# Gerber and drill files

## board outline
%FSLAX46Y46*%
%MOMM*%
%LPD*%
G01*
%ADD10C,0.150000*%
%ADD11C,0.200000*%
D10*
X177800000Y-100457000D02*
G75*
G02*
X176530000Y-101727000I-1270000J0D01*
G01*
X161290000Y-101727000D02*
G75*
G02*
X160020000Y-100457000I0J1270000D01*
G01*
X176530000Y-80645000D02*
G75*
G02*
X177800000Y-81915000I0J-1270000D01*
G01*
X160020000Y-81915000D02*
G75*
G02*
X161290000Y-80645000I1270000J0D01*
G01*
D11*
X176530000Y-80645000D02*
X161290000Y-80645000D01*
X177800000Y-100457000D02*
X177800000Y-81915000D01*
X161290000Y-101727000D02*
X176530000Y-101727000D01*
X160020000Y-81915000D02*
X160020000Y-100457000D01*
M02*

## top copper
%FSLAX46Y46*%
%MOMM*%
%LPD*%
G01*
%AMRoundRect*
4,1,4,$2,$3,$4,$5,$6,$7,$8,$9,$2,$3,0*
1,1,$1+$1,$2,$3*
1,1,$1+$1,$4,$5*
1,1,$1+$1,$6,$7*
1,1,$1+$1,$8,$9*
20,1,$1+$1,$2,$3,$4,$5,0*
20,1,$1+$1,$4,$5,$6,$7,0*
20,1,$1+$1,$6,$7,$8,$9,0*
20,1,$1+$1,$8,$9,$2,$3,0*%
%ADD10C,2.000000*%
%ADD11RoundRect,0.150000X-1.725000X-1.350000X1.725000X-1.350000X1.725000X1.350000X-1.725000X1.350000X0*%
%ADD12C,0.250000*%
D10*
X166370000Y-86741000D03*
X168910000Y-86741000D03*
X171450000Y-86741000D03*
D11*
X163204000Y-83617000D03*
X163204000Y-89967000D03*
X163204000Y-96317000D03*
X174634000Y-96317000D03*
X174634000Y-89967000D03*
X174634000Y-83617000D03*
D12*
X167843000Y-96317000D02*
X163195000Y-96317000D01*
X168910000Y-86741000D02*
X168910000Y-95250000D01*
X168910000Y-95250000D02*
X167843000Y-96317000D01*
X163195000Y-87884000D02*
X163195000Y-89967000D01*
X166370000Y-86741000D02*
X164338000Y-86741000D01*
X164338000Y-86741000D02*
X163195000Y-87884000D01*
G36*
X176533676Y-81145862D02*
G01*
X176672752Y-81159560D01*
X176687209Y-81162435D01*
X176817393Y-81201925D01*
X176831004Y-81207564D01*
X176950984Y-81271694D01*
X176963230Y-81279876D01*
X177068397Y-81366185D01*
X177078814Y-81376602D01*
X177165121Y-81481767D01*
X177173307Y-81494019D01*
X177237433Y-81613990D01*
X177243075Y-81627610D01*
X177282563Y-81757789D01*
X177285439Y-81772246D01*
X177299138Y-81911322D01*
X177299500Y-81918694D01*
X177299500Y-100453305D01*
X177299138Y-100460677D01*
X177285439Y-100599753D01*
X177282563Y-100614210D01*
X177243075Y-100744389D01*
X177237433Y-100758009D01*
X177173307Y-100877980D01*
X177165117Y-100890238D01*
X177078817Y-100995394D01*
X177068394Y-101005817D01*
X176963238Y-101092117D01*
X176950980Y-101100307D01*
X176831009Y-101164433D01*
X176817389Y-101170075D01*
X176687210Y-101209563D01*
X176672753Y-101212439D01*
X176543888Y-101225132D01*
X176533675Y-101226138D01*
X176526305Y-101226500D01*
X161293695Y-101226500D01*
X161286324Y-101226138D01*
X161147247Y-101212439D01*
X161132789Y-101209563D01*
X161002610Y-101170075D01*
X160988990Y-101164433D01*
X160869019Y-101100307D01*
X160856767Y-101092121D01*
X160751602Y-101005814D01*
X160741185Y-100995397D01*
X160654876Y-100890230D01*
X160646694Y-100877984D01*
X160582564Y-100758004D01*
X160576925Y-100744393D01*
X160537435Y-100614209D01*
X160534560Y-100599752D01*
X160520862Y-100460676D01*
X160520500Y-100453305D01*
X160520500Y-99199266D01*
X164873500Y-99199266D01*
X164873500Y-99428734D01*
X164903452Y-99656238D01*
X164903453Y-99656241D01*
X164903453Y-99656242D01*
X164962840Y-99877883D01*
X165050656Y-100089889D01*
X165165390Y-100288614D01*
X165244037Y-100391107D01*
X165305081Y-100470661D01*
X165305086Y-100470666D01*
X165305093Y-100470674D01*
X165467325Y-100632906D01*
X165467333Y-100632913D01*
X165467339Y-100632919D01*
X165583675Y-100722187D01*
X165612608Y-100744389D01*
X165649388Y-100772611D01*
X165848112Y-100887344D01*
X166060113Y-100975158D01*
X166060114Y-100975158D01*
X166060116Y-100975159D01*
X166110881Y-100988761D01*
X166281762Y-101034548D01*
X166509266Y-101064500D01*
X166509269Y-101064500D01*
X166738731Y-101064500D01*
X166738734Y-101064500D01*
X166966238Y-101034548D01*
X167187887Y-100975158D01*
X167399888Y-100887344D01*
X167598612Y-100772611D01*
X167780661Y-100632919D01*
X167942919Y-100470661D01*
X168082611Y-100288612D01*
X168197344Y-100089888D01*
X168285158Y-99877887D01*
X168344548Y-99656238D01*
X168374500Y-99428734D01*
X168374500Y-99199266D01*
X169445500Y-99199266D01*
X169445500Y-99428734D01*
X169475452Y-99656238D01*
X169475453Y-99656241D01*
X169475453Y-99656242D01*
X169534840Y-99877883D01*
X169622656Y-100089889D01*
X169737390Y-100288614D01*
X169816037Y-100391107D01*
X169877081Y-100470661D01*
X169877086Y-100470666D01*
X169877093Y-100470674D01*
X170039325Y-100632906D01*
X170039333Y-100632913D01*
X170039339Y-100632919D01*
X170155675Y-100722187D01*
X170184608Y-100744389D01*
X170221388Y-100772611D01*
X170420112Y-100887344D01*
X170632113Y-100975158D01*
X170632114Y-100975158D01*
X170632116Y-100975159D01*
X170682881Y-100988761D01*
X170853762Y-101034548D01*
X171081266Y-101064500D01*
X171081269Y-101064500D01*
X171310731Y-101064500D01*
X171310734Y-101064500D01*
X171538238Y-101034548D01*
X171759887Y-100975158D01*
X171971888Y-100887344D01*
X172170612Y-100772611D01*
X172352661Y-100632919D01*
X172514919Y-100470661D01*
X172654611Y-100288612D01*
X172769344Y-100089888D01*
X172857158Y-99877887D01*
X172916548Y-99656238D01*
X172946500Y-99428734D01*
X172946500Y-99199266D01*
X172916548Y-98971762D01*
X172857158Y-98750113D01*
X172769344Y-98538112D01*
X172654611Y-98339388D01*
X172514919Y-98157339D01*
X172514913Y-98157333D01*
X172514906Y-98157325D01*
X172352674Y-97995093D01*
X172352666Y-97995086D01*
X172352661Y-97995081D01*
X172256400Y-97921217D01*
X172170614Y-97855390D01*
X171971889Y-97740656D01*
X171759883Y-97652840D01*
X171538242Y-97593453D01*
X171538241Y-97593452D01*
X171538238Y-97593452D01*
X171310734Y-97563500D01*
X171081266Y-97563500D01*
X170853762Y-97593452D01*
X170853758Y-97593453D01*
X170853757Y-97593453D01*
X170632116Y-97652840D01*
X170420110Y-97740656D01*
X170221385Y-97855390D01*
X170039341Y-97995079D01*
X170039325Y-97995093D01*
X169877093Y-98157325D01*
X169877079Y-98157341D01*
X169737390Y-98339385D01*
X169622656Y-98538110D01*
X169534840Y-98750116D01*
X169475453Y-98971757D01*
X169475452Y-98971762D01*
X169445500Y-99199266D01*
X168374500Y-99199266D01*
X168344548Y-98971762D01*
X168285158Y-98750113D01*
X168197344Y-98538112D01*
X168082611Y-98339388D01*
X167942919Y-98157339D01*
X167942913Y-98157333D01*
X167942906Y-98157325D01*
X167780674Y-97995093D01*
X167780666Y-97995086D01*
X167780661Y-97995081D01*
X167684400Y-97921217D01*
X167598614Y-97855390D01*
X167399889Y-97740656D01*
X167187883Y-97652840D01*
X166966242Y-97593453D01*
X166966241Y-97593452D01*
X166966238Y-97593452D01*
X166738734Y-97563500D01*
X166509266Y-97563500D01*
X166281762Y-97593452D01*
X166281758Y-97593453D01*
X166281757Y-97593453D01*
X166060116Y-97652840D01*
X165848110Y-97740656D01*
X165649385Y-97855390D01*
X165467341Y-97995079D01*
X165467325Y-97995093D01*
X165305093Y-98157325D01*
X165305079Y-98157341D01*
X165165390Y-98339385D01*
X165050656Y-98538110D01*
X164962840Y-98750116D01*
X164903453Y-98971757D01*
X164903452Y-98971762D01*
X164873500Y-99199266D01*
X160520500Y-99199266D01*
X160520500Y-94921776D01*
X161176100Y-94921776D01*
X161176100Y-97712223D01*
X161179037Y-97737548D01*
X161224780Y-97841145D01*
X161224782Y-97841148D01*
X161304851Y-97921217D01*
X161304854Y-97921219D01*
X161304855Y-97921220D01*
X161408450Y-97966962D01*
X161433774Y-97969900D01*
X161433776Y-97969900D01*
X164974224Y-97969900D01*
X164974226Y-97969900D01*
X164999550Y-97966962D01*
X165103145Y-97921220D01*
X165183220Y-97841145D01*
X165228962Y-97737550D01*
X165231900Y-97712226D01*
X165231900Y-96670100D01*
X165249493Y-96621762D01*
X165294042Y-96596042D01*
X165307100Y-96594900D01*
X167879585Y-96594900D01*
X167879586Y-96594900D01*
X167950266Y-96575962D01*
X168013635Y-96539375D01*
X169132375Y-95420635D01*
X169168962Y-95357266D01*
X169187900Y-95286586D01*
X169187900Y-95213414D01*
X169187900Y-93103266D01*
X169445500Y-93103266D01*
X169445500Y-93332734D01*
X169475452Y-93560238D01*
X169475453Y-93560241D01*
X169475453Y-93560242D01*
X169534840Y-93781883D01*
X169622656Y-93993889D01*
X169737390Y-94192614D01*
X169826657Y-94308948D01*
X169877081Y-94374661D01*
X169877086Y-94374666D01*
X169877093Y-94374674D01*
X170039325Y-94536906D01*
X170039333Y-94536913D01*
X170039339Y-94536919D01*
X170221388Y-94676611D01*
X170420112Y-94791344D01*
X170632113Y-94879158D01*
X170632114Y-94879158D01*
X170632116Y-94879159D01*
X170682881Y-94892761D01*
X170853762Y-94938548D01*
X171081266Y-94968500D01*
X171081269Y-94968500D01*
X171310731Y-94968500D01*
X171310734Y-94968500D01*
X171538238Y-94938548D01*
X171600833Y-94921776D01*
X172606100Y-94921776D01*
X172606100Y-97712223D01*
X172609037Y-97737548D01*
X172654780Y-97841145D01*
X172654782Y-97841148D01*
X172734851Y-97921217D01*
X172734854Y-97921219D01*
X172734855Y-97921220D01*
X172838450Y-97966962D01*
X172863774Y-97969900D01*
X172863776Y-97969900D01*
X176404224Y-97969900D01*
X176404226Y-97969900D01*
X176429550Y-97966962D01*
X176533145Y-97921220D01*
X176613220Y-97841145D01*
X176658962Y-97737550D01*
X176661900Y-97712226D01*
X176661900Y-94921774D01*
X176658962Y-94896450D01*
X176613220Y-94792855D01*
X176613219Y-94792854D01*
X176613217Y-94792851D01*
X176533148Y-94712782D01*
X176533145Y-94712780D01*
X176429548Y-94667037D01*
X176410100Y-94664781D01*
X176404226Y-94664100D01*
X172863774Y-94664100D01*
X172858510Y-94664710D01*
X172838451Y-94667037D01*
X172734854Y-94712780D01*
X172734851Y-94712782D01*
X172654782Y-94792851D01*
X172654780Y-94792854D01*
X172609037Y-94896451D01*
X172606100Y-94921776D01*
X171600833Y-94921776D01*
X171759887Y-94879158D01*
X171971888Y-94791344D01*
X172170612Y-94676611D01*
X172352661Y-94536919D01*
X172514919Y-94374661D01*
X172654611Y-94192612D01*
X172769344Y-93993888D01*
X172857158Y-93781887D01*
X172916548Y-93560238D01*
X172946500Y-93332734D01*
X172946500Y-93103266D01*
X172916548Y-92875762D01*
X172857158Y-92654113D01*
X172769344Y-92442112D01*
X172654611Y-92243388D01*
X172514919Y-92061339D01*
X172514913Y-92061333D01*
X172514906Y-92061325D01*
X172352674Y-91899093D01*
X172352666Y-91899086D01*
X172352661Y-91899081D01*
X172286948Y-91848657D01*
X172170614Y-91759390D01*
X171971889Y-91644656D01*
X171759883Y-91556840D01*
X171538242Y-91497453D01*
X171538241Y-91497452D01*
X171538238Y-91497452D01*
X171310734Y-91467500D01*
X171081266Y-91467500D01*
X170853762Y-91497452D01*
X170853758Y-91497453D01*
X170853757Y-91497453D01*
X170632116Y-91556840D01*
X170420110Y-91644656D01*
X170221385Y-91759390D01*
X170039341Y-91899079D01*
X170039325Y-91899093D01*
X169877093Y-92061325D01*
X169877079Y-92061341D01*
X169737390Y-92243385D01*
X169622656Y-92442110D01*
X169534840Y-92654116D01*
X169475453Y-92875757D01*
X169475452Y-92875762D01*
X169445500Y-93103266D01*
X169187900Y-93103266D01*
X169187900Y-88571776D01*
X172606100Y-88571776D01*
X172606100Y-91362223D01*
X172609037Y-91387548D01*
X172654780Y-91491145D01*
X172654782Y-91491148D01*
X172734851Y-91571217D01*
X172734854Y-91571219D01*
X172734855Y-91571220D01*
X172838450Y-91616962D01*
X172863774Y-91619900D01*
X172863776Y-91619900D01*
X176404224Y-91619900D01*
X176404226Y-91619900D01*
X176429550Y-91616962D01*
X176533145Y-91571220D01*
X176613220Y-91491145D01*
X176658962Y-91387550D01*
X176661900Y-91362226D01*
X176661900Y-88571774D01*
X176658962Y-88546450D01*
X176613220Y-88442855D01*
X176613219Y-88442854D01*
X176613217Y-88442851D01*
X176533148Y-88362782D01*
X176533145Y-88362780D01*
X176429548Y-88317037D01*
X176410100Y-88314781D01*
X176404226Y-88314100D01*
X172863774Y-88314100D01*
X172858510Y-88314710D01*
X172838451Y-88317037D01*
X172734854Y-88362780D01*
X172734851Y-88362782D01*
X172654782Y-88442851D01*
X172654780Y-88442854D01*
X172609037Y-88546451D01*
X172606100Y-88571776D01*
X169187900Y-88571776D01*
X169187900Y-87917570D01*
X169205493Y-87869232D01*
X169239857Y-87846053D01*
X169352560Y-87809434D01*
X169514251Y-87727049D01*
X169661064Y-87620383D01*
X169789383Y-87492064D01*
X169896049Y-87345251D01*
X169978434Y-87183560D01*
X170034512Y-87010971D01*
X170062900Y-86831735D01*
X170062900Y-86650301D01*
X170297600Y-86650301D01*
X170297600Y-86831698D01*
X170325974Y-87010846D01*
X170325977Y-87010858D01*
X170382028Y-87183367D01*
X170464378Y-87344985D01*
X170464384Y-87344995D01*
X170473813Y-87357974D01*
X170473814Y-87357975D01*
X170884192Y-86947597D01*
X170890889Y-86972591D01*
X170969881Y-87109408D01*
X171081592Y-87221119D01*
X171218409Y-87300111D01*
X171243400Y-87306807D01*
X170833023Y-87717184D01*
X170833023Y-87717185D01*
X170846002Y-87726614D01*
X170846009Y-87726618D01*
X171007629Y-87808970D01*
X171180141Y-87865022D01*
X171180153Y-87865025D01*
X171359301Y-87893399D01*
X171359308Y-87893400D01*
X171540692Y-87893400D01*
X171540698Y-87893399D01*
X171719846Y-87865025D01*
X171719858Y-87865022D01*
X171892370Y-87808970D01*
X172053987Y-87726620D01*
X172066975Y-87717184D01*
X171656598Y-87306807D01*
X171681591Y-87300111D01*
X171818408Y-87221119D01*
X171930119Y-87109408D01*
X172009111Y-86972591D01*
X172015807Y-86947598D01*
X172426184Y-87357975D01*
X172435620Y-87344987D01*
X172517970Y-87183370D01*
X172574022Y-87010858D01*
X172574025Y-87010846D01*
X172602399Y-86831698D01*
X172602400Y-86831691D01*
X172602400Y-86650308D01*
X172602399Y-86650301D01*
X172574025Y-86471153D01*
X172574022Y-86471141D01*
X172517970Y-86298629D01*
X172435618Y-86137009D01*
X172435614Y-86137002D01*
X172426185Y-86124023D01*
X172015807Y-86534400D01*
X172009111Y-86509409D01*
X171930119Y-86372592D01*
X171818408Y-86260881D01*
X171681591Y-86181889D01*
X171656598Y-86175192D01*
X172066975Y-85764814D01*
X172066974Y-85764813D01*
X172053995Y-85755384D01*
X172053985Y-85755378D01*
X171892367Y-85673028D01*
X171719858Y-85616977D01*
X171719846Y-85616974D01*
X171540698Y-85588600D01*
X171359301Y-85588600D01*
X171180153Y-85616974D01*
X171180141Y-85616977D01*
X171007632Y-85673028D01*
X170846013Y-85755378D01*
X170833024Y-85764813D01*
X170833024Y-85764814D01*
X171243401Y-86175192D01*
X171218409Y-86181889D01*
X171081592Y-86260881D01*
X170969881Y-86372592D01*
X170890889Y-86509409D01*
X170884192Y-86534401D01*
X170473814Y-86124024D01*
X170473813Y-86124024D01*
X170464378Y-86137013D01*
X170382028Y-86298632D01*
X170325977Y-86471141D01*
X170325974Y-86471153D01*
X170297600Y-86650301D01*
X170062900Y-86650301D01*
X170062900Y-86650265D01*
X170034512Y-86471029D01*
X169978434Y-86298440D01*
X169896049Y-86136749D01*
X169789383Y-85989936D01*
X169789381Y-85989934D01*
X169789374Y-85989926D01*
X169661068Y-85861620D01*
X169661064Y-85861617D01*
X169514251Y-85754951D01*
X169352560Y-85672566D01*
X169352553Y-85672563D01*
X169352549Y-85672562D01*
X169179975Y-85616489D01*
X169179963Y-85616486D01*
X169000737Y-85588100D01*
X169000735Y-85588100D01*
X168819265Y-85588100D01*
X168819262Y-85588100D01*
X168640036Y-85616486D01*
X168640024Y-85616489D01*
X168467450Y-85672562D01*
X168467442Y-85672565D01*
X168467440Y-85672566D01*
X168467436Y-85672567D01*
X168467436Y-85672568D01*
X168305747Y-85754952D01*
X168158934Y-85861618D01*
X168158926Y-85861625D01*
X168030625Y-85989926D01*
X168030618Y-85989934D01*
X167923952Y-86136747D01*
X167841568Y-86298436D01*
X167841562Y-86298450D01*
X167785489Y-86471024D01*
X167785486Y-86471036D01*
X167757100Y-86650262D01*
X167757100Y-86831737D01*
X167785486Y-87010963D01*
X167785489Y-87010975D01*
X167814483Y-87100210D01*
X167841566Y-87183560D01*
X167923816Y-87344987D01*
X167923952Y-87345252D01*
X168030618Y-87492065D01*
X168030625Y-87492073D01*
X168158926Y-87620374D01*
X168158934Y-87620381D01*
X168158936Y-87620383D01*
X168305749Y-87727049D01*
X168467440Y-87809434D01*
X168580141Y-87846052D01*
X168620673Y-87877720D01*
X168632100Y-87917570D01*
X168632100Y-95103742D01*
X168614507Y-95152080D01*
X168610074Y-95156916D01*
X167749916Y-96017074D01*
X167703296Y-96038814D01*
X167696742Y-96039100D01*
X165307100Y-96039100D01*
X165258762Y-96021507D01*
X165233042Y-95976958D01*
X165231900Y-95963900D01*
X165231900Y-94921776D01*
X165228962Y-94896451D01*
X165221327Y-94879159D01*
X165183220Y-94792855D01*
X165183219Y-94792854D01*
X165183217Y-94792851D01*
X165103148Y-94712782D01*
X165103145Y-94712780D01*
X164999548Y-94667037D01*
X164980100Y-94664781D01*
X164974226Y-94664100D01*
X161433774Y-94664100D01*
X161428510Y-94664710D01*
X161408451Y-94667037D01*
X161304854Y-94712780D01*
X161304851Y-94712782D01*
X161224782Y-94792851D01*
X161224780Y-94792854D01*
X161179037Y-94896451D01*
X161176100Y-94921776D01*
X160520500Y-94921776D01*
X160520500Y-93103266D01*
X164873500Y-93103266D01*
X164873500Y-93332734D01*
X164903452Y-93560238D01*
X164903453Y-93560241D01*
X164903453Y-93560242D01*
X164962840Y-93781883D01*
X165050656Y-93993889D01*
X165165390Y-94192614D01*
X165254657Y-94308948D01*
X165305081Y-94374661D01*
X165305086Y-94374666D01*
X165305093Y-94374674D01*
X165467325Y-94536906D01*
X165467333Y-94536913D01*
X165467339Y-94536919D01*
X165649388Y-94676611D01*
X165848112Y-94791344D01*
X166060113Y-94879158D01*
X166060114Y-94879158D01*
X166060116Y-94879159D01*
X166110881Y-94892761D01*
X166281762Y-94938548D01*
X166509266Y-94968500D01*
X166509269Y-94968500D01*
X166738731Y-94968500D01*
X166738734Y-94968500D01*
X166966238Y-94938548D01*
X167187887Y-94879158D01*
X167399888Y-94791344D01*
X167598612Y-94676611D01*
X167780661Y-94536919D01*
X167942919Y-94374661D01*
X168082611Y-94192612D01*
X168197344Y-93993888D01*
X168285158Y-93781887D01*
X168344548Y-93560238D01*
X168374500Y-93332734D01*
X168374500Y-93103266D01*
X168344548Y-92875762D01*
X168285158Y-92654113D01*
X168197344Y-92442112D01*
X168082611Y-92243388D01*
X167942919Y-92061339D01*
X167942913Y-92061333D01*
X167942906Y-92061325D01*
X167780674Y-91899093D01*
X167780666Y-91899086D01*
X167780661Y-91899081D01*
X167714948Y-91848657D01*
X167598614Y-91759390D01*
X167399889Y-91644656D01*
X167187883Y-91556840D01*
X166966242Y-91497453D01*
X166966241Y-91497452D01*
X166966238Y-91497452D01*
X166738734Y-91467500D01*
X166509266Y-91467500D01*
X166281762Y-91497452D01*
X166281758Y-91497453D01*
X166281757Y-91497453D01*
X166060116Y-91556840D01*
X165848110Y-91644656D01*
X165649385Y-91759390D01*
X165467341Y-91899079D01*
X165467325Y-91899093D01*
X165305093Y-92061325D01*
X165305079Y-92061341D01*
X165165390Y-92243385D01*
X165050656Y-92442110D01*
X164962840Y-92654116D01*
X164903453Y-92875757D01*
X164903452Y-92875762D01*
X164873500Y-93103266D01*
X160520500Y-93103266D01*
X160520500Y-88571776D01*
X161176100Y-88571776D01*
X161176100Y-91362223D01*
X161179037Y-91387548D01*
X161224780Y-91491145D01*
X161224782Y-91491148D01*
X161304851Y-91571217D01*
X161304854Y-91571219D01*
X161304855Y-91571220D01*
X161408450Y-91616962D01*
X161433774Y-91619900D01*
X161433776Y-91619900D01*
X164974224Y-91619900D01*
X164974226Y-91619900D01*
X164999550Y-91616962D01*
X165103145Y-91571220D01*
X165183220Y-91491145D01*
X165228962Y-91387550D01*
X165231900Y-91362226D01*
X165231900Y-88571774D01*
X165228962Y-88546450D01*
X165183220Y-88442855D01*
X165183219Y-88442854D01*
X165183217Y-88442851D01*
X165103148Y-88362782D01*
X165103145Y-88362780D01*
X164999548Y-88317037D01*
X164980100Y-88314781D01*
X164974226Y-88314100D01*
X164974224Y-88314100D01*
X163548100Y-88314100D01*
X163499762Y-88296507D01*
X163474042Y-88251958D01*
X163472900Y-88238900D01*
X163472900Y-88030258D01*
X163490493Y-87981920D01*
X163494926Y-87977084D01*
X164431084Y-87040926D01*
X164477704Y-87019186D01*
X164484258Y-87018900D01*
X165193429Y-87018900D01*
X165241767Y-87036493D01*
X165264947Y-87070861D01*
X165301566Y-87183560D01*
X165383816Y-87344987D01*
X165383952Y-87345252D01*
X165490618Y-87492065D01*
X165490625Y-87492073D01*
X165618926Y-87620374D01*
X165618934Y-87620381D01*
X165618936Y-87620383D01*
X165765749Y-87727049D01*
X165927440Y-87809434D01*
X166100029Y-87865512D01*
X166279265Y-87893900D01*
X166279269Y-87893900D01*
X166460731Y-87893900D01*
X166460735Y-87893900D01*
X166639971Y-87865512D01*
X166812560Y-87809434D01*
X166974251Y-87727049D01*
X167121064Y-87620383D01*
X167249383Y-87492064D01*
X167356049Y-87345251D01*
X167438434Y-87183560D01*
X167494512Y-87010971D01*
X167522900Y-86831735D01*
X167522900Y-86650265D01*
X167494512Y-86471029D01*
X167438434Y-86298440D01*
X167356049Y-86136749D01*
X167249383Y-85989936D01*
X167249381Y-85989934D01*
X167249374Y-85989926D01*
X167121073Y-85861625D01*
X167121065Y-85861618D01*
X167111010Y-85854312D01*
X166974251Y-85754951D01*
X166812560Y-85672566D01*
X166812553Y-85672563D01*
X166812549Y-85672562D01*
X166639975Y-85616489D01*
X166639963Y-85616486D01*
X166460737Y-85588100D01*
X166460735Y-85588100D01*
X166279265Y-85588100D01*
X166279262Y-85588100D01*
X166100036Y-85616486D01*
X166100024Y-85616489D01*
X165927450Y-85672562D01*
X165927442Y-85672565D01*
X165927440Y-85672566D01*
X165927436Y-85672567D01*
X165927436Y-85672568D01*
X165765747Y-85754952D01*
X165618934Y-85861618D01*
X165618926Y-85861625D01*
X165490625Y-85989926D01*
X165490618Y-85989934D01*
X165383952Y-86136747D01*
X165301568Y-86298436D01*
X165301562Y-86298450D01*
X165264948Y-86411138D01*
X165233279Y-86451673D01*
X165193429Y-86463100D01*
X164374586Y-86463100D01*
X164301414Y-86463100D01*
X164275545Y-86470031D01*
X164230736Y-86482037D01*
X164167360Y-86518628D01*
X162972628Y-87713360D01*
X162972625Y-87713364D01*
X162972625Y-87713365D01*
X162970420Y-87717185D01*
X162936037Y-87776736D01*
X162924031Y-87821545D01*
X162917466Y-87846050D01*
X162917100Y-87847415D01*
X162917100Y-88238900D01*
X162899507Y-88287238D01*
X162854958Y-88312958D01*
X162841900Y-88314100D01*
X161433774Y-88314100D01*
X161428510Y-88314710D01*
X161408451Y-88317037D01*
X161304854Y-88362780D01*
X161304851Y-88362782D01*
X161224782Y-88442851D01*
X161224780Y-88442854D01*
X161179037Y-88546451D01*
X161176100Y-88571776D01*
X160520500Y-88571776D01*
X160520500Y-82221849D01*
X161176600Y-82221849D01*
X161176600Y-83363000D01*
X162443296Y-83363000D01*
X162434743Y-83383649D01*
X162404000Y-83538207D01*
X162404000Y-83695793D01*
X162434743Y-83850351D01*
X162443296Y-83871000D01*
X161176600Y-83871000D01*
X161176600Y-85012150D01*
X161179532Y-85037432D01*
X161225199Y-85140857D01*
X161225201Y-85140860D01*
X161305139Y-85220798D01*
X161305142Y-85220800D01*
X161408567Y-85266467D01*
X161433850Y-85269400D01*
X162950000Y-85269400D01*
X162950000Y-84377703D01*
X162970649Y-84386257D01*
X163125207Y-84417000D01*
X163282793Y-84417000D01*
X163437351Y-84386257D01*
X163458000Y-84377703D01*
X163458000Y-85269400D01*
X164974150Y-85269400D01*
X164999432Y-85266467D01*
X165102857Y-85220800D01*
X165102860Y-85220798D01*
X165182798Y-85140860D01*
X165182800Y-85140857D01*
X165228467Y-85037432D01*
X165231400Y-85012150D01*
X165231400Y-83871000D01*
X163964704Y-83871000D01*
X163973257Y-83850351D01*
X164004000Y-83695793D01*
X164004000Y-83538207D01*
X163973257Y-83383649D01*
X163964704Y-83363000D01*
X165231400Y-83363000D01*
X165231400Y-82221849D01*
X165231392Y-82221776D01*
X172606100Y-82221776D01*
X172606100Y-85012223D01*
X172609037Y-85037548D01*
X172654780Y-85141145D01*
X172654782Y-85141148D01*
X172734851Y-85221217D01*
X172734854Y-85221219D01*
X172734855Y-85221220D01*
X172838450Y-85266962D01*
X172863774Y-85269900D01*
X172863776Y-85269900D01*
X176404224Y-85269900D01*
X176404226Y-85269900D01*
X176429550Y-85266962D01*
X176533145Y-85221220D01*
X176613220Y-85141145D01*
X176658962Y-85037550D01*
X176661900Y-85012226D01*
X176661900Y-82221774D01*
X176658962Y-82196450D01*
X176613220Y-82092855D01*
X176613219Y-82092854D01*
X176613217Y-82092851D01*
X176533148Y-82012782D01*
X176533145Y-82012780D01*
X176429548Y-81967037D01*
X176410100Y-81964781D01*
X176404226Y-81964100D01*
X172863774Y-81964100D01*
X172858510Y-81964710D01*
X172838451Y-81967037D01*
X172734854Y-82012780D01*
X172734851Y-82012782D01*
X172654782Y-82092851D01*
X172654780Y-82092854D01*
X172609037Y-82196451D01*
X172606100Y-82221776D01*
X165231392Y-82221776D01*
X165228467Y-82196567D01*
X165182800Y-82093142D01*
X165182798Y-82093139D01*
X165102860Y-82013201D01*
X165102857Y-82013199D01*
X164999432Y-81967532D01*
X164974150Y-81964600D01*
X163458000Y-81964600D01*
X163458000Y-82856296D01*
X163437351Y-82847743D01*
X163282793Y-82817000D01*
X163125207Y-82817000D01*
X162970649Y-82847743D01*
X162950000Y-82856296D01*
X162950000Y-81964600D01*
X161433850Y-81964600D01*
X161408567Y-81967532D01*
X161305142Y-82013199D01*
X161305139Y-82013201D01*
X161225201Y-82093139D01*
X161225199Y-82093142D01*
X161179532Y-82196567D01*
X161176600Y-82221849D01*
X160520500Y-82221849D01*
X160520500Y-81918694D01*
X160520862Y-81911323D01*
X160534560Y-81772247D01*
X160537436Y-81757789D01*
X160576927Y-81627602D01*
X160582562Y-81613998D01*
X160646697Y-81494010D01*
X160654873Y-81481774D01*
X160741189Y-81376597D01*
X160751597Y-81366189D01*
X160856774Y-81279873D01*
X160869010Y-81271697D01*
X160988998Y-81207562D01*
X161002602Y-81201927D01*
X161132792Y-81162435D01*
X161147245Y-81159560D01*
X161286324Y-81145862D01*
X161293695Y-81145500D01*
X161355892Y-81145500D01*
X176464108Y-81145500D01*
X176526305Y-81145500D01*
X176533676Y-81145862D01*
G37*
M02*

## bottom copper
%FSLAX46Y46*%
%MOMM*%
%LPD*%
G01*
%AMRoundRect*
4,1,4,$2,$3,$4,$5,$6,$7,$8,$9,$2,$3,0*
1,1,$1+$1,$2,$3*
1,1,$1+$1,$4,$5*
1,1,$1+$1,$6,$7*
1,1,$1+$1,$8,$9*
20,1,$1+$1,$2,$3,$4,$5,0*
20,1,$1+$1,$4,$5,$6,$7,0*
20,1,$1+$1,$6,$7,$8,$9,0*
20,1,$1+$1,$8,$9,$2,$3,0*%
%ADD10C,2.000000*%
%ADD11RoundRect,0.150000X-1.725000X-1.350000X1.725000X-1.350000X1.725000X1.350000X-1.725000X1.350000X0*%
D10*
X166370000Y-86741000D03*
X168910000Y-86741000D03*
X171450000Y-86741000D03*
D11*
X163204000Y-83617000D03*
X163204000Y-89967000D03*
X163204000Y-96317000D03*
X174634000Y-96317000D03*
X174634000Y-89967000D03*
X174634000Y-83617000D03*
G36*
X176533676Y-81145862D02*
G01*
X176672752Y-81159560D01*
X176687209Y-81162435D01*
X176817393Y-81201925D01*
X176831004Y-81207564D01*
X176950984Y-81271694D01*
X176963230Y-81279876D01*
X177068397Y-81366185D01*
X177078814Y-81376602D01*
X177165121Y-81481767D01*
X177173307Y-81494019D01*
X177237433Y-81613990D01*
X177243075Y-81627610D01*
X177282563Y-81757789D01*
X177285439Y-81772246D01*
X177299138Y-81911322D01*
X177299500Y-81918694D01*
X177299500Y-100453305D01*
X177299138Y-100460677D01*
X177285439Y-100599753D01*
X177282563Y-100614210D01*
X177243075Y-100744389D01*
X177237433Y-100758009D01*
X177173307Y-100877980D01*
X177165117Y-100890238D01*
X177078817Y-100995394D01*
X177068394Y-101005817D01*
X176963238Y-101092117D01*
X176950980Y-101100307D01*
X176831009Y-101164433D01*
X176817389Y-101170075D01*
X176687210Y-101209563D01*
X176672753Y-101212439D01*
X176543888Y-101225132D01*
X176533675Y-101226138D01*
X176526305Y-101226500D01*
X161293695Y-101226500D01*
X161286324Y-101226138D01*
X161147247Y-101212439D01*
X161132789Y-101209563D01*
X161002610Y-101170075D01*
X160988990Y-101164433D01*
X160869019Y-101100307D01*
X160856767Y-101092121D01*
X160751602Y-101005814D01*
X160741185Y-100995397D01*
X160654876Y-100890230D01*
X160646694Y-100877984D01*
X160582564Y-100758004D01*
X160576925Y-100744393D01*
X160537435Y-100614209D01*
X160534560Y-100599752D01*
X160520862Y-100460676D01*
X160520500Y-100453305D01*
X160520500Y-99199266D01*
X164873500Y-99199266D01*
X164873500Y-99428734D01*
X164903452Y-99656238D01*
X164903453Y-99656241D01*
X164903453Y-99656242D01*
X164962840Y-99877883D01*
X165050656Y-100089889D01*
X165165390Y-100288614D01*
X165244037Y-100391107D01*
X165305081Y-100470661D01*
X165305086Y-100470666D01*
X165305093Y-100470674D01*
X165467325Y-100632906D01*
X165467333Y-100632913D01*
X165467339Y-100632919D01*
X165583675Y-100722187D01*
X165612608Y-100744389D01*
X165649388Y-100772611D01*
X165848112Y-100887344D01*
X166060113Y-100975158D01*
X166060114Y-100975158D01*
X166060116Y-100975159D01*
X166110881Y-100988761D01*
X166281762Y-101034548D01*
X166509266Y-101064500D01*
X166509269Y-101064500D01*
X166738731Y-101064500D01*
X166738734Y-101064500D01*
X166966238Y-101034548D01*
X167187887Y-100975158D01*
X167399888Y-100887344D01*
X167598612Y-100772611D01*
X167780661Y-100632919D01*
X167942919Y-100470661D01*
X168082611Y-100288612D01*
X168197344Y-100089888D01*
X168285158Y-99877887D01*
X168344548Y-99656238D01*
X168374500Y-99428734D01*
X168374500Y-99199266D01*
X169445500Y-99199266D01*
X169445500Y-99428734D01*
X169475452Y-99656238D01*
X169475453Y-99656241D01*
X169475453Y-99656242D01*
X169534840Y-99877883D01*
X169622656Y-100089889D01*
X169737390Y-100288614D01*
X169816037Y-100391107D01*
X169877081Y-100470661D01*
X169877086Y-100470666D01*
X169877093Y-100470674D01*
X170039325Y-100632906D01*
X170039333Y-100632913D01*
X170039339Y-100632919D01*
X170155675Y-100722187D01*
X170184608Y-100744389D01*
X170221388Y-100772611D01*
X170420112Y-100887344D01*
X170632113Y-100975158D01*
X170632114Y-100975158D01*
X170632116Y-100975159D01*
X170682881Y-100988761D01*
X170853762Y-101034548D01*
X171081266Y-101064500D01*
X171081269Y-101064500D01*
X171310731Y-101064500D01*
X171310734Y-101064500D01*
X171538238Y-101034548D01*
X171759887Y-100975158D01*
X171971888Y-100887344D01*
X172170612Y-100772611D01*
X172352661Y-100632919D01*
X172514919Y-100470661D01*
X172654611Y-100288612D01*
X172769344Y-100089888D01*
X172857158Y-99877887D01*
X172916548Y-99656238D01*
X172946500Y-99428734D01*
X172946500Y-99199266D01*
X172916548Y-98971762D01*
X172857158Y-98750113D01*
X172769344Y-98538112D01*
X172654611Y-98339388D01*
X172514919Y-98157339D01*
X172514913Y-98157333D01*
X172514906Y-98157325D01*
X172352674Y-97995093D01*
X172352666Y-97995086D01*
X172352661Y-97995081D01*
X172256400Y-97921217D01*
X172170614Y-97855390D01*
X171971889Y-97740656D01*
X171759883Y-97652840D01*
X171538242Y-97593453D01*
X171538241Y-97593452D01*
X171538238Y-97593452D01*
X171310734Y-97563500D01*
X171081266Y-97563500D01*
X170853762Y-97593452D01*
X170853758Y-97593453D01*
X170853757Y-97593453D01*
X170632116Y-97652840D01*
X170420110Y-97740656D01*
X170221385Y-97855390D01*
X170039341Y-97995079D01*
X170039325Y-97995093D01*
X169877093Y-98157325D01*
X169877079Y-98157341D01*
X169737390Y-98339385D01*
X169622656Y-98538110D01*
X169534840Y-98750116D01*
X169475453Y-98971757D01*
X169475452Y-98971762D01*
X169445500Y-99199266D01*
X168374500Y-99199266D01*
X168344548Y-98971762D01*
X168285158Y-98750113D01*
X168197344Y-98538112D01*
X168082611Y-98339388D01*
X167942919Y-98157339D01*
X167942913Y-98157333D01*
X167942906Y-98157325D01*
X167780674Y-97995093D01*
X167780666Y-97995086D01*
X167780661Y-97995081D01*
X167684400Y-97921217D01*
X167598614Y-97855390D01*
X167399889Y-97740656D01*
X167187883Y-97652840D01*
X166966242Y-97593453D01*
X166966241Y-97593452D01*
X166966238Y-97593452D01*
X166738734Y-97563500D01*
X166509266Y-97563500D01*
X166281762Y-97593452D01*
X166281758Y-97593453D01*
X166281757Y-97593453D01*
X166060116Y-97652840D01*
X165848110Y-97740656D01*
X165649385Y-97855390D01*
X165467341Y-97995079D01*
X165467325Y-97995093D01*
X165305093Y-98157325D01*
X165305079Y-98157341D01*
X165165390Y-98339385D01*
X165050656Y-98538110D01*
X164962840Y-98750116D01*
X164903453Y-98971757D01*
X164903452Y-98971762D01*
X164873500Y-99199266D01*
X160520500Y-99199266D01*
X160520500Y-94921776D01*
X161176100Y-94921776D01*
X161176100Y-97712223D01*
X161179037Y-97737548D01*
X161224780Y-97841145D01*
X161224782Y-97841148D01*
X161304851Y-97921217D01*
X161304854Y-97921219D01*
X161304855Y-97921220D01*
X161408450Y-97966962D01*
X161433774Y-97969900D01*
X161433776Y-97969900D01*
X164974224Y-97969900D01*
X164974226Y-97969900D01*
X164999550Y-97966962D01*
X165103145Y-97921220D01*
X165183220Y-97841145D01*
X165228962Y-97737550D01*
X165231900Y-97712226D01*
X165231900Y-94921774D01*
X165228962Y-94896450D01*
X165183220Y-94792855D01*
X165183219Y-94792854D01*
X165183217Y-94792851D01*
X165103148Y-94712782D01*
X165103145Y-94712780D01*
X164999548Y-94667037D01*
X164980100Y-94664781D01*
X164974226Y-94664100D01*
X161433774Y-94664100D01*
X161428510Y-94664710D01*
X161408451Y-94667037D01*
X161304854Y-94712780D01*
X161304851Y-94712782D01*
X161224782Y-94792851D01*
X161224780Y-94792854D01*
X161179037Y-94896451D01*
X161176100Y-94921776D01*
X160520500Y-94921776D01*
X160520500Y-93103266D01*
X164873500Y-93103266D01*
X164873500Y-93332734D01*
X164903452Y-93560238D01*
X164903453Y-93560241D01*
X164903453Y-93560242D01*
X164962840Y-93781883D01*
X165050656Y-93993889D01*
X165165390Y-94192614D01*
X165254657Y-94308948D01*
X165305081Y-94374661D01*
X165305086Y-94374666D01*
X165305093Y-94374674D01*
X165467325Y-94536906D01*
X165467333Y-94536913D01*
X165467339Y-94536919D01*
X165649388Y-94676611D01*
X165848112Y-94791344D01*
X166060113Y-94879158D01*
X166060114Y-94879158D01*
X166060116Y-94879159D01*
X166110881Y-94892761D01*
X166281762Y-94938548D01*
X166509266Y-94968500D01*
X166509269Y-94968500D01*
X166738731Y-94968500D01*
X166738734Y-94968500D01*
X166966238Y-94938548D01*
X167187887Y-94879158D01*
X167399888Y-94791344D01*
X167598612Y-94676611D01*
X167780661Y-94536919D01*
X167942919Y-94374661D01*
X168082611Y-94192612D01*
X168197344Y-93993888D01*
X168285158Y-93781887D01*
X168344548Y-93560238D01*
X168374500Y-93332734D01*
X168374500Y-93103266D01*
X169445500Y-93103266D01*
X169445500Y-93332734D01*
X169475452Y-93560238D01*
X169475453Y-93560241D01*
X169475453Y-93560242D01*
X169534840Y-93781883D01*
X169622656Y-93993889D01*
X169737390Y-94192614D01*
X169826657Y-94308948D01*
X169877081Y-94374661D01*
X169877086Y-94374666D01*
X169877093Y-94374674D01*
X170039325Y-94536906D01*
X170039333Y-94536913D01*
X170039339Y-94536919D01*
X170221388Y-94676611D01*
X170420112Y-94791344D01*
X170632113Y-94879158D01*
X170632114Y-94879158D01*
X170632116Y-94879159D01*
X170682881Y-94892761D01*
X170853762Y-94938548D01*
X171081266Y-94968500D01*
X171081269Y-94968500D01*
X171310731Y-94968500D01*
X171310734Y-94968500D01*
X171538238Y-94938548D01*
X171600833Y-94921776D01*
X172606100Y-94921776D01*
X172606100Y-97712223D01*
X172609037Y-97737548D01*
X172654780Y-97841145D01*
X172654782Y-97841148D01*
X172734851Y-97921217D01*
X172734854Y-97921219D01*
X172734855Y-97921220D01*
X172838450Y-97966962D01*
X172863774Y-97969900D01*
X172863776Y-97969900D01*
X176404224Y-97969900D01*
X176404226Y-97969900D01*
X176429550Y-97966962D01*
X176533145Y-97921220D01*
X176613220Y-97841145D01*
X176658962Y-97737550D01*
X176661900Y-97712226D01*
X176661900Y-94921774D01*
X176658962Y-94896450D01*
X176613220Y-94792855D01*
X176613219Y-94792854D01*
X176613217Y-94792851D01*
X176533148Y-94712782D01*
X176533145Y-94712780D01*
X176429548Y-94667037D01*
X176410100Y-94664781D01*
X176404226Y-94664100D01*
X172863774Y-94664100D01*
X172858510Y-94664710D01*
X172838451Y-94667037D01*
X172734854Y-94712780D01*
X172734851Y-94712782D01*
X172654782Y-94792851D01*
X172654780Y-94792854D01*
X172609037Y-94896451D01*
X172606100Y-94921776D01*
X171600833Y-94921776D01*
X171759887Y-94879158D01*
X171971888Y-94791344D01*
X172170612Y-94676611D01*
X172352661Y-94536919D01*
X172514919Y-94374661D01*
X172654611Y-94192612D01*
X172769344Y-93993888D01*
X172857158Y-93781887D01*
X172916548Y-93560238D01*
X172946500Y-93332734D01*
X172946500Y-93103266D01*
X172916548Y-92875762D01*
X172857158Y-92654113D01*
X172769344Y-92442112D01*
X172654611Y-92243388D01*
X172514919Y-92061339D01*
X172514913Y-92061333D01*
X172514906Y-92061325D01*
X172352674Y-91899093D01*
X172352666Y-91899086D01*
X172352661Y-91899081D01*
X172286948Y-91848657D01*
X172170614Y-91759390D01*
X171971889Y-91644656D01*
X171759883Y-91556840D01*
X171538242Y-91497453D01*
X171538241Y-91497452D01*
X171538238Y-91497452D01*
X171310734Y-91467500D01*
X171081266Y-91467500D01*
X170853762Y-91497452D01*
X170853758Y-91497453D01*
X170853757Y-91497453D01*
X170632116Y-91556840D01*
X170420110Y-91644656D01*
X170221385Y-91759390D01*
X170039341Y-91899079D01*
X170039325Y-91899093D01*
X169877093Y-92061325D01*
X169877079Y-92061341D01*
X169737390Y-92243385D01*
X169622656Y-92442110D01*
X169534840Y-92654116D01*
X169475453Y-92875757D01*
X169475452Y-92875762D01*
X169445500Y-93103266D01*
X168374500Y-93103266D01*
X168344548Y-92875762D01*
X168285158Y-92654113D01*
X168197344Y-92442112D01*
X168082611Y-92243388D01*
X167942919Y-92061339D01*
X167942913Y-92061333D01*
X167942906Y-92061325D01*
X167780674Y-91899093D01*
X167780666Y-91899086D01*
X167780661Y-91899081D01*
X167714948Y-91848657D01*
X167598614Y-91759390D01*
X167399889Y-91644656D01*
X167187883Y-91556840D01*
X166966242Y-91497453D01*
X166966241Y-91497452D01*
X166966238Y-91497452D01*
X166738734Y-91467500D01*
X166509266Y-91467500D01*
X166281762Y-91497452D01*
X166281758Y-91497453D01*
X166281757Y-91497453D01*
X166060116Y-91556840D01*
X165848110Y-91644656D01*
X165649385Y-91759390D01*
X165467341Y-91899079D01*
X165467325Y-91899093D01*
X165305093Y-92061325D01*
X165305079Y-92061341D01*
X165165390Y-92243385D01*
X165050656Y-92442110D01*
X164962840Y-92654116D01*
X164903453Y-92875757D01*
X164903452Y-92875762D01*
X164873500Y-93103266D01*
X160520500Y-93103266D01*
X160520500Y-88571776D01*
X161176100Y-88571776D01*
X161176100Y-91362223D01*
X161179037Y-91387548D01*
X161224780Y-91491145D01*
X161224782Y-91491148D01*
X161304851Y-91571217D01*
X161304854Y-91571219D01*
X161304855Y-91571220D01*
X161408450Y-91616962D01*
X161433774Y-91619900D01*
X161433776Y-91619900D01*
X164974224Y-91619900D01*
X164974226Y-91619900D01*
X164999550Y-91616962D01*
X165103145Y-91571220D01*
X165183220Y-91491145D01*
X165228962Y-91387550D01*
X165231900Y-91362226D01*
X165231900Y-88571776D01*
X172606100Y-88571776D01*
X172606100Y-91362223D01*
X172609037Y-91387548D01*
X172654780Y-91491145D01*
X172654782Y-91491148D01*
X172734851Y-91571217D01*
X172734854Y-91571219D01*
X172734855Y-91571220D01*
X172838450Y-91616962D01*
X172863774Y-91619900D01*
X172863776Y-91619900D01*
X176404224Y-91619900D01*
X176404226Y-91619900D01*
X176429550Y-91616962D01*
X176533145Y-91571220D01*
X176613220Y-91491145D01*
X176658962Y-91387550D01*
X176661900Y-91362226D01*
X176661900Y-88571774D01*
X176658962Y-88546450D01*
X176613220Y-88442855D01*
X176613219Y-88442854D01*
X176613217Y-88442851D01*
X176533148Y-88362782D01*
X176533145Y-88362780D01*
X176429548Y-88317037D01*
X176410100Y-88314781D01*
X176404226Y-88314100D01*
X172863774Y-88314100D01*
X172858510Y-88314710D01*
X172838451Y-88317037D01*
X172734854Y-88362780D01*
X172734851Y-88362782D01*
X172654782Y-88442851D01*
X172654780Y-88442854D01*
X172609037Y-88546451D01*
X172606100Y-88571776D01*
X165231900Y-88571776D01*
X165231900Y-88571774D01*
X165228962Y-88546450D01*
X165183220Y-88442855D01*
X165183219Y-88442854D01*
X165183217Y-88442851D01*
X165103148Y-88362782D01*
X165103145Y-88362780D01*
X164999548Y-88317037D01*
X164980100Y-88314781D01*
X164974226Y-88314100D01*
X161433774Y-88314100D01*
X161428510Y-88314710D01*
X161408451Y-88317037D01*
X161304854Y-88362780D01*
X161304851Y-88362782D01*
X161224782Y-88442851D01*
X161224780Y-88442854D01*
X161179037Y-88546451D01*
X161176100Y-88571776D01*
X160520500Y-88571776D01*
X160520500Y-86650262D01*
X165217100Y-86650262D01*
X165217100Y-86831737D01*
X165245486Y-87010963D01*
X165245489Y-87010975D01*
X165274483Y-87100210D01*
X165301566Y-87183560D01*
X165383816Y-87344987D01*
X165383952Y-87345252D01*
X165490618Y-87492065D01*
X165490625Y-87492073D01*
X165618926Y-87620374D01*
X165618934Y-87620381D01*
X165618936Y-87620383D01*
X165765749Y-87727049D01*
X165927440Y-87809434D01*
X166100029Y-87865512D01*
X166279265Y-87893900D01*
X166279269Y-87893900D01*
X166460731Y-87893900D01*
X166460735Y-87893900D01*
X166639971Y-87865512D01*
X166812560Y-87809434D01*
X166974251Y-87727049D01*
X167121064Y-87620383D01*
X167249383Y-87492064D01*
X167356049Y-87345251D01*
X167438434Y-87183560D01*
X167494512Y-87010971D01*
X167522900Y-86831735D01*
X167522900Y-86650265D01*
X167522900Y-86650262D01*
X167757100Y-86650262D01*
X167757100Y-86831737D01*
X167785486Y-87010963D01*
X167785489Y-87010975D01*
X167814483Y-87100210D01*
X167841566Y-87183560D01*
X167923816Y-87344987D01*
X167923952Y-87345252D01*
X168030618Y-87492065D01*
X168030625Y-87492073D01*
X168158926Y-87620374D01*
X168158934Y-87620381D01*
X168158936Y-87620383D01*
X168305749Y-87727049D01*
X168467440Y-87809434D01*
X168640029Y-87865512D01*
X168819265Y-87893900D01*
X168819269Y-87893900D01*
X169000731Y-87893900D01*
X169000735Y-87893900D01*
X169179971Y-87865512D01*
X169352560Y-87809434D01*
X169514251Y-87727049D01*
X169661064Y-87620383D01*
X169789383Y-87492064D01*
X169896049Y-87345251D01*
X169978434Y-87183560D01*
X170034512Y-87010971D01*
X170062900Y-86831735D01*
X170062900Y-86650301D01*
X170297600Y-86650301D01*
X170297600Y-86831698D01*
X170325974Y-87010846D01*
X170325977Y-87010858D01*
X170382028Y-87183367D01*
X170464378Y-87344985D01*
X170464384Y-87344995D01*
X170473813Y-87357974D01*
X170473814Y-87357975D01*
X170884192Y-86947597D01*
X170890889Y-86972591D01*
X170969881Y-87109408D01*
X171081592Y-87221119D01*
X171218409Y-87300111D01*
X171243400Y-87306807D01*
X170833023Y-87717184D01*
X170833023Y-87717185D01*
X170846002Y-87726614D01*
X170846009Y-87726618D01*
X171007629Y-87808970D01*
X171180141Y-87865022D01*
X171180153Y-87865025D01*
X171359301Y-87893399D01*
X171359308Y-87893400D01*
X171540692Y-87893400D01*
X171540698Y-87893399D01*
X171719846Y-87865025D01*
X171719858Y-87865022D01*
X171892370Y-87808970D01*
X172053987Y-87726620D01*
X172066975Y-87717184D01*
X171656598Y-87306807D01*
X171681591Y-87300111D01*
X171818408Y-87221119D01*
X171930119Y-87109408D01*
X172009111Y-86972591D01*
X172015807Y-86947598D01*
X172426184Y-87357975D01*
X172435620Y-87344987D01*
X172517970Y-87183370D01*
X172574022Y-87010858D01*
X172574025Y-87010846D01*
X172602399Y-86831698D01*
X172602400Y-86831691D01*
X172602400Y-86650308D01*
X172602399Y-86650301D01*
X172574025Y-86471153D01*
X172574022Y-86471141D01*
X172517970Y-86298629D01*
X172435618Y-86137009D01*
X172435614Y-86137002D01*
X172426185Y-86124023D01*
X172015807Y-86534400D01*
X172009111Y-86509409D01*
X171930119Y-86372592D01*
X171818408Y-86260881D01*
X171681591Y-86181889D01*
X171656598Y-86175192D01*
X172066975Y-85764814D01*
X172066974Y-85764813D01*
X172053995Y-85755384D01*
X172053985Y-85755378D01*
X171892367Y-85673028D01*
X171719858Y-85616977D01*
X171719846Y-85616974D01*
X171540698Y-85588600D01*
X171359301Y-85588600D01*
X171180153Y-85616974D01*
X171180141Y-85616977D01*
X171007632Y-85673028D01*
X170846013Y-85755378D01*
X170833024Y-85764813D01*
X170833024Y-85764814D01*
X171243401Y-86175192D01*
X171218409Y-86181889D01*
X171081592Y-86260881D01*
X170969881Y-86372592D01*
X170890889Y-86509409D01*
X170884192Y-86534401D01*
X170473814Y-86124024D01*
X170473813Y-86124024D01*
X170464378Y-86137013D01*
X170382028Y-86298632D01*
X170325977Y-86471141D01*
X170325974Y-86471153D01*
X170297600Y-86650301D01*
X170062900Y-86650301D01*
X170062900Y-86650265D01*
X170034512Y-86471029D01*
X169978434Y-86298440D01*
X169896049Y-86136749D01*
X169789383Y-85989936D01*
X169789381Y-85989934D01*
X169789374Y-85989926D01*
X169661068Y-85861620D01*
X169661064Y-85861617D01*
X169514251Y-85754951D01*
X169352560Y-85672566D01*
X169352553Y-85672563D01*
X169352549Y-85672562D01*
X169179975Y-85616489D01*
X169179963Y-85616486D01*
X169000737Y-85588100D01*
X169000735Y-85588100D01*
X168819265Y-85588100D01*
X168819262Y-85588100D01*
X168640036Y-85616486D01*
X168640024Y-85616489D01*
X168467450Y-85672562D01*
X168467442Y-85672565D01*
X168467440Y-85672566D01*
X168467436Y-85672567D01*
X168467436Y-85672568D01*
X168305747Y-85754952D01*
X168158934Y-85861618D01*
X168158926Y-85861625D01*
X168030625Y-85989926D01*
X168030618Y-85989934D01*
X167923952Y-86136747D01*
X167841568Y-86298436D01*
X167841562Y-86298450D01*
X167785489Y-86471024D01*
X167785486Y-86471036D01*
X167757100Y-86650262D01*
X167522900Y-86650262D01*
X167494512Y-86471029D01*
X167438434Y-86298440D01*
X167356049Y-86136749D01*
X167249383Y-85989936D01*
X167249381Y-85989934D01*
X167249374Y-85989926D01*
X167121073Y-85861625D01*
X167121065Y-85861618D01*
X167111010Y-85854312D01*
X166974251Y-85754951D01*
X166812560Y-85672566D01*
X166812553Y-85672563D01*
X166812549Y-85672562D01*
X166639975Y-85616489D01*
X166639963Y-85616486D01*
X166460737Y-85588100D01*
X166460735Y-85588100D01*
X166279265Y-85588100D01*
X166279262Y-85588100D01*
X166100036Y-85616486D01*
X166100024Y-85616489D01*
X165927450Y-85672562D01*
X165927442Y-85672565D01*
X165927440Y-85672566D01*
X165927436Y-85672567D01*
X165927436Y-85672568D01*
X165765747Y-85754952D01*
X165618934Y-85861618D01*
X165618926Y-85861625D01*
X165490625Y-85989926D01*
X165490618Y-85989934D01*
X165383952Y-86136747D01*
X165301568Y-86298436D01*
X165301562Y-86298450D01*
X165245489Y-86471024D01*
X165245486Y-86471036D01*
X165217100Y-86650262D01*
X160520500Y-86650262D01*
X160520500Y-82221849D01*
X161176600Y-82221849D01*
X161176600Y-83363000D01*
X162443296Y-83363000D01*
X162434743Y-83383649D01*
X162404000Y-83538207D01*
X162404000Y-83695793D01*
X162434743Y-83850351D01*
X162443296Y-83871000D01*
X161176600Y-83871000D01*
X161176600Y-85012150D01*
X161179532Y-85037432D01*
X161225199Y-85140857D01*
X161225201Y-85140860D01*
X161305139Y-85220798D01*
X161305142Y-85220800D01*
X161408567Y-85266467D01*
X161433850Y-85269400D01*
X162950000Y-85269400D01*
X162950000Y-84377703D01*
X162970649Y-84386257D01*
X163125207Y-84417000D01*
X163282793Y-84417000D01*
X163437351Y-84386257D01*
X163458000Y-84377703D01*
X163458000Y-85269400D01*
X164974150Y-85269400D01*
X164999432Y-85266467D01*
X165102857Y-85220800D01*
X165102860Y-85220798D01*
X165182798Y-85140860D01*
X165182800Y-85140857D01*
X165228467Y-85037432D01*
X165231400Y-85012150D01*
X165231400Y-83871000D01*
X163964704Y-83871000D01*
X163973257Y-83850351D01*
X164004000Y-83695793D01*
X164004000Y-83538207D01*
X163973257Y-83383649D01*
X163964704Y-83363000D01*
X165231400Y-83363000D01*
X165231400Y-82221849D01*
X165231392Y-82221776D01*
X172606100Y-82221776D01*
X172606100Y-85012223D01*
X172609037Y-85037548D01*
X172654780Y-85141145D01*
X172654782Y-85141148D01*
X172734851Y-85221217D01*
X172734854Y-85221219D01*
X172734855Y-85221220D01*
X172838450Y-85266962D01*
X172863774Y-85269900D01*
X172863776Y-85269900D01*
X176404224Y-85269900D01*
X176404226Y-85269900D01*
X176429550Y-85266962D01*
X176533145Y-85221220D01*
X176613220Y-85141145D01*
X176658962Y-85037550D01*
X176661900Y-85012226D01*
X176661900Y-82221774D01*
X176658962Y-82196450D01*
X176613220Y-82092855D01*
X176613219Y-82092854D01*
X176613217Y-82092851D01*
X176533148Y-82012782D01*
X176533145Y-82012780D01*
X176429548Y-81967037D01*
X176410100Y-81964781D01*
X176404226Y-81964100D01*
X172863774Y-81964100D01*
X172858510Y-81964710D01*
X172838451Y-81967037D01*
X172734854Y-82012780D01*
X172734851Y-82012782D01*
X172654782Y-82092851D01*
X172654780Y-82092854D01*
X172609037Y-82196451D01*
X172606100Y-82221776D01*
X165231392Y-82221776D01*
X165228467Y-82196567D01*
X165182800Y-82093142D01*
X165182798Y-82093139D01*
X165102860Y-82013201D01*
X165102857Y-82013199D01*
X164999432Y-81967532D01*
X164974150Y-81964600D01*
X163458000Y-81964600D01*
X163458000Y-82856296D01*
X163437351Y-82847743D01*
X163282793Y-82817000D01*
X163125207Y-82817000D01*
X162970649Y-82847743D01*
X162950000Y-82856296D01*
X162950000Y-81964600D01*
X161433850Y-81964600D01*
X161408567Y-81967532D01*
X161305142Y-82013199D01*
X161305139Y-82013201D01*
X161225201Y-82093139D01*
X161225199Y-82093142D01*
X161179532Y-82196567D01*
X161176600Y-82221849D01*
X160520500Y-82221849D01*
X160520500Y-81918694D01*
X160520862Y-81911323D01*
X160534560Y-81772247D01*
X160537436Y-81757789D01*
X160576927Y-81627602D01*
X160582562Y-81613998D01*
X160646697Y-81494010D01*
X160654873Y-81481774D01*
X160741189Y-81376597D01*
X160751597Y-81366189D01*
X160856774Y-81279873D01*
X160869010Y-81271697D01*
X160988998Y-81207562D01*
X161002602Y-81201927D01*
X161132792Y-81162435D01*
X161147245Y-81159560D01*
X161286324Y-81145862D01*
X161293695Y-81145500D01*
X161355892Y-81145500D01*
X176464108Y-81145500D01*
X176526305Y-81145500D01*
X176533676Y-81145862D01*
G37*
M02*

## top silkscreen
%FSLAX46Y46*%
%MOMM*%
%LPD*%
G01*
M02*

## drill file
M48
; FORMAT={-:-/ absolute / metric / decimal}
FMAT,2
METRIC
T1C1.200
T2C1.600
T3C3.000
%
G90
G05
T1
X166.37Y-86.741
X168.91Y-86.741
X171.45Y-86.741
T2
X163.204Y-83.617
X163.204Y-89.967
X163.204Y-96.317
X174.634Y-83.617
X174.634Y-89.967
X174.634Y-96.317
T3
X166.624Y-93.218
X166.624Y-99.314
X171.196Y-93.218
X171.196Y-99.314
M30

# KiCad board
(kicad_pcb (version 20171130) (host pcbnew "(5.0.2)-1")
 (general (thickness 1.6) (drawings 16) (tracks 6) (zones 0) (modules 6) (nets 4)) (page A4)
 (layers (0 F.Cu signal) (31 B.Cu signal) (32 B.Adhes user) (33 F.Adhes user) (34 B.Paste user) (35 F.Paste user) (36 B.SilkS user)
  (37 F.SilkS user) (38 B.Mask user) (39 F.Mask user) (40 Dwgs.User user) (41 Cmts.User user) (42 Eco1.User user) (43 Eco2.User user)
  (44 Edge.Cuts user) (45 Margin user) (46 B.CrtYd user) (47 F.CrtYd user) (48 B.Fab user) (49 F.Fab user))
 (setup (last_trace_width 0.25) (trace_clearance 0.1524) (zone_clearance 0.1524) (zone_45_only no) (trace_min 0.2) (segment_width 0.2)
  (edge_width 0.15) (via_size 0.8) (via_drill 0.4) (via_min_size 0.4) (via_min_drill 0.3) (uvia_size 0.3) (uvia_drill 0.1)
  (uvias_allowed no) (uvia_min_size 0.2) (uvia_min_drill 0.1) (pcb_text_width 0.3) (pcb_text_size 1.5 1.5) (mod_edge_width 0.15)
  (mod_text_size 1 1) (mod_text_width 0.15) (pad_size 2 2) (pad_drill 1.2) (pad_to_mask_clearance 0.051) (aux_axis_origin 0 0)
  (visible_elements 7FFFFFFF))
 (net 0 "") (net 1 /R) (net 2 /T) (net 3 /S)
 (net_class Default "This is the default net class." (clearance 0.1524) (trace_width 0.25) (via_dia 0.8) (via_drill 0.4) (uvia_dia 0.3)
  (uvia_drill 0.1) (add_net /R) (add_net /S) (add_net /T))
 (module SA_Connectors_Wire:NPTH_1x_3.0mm (layer F.Cu) (at 171.196 99.314)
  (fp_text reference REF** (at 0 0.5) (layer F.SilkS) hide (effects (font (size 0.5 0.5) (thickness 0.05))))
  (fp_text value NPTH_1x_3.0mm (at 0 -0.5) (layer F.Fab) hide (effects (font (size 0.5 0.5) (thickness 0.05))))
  (pad "" np_thru_hole circle (at 0 0) (size 3 3) (drill 3) (layers *.Cu *.Mask)))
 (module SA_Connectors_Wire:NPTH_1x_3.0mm (layer F.Cu) (at 166.624 99.314)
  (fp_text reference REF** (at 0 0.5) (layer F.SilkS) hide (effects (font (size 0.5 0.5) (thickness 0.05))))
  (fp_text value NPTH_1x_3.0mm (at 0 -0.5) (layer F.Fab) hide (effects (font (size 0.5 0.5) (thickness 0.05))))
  (pad "" np_thru_hole circle (at 0 0) (size 3 3) (drill 3) (layers *.Cu *.Mask)))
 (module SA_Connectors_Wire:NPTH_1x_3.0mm (layer F.Cu) (at 171.196 93.218)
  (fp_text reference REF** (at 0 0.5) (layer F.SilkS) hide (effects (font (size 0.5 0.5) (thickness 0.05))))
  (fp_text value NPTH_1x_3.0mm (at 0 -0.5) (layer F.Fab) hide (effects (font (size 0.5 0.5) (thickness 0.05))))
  (pad "" np_thru_hole circle (at 0 0) (size 3 3) (drill 3) (layers *.Cu *.Mask)))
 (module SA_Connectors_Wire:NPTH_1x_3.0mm (layer F.Cu) (at 166.624 93.218)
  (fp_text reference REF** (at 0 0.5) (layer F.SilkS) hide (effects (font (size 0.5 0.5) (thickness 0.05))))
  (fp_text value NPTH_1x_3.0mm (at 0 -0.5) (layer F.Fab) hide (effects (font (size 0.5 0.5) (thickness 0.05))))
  (pad "" np_thru_hole circle (at 0 0) (size 3 3) (drill 3) (layers *.Cu *.Mask)))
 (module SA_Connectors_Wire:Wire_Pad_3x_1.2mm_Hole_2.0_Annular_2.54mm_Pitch (layer F.Cu) (at 168.91 86.741)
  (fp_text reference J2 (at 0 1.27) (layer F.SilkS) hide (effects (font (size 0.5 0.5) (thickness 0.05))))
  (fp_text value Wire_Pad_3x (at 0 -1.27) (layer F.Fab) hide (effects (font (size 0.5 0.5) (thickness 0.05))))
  (pad 1 thru_hole circle (at -2.54 0) (size 2 2) (drill 1.2) (layers *.Cu *.Mask) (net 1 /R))
  (pad 2 thru_hole circle (at 0 0) (size 2 2) (drill 1.2) (layers *.Cu *.Mask) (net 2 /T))
  (pad 3 thru_hole circle (at 2.54 0) (size 2 2) (drill 1.2) (layers *.Cu *.Mask) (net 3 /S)))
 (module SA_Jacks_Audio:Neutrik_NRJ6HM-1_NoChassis (layer F.Cu) (at 170.434 78.867)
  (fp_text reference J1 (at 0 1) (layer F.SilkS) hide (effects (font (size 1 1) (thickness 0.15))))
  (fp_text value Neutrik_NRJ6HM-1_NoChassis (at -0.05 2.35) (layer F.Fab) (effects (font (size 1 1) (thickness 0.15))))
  (pad S thru_hole roundrect (at -7.23 4.75) (size 3.75 3) (drill 1.6) (layers *.Cu *.Mask) (roundrect_rratio 0.05) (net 3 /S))
  (pad R thru_hole roundrect (at -7.23 11.1) (size 3.75 3) (drill 1.6) (layers *.Cu *.Mask) (roundrect_rratio 0.05) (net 1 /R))
  (pad T thru_hole roundrect (at -7.23 17.45) (size 3.75 3) (drill 1.6) (layers *.Cu *.Mask) (roundrect_rratio 0.05) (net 2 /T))
  (pad TN thru_hole roundrect (at 4.2 17.45) (size 3.75 3) (drill 1.6) (layers *.Cu *.Mask) (roundrect_rratio 0.05))
  (pad RN thru_hole roundrect (at 4.2 11.1) (size 3.75 3) (drill 1.6) (layers *.Cu *.Mask) (roundrect_rratio 0.05))
  (pad SN thru_hole roundrect (at 4.2 4.75) (size 3.75 3) (drill 1.6) (layers *.Cu *.Mask) (roundrect_rratio 0.05)))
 (gr_arc (start 176.53 100.457) (end 176.53 101.727) (angle -90) (layer Edge.Cuts) (width 0.15))
 (gr_arc (start 161.29 100.457) (end 160.02 100.457) (angle -90) (layer Edge.Cuts) (width 0.15))
 (gr_arc (start 176.53 81.915) (end 177.8 81.915) (angle -90) (layer Edge.Cuts) (width 0.15))
 (gr_arc (start 161.29 81.915) (end 161.29 80.645) (angle -90) (layer Edge.Cuts) (width 0.15))
 (gr_line (start 176.53 80.645) (end 161.29 80.645) (layer Edge.Cuts) (width 0.2))
 (gr_line (start 177.8 100.457) (end 177.8 81.915) (layer Edge.Cuts) (width 0.2))
 (gr_line (start 161.29 101.727) (end 176.53 101.727) (layer Edge.Cuts) (width 0.2))
 (gr_line (start 160.02 81.915) (end 160.02 100.457) (layer Edge.Cuts) (width 0.2))
 (segment (start 167.843 96.317) (end 163.195 96.317) (width 0.25) (layer F.Cu) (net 2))
 (segment (start 168.91 86.741) (end 168.91 95.25) (width 0.25) (layer F.Cu) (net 2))
 (segment (start 168.91 95.25) (end 167.843 96.317) (width 0.25) (layer F.Cu) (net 2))
 (segment (start 163.195 87.884) (end 163.195 89.967) (width 0.25) (layer F.Cu) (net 1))
 (segment (start 166.37 86.741) (end 164.338 86.741) (width 0.25) (layer F.Cu) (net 1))
 (segment (start 164.338 86.741) (end 163.195 87.884) (width 0.25) (layer F.Cu) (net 1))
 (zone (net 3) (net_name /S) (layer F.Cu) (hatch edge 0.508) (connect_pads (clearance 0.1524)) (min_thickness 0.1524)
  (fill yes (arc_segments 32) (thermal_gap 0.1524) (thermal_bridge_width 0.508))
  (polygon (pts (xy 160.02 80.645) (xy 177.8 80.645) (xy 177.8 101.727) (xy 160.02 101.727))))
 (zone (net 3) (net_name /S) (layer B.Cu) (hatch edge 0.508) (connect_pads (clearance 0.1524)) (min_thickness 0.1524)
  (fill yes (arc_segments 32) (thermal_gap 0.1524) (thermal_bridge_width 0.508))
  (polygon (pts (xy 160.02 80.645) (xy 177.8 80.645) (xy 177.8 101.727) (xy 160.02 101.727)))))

